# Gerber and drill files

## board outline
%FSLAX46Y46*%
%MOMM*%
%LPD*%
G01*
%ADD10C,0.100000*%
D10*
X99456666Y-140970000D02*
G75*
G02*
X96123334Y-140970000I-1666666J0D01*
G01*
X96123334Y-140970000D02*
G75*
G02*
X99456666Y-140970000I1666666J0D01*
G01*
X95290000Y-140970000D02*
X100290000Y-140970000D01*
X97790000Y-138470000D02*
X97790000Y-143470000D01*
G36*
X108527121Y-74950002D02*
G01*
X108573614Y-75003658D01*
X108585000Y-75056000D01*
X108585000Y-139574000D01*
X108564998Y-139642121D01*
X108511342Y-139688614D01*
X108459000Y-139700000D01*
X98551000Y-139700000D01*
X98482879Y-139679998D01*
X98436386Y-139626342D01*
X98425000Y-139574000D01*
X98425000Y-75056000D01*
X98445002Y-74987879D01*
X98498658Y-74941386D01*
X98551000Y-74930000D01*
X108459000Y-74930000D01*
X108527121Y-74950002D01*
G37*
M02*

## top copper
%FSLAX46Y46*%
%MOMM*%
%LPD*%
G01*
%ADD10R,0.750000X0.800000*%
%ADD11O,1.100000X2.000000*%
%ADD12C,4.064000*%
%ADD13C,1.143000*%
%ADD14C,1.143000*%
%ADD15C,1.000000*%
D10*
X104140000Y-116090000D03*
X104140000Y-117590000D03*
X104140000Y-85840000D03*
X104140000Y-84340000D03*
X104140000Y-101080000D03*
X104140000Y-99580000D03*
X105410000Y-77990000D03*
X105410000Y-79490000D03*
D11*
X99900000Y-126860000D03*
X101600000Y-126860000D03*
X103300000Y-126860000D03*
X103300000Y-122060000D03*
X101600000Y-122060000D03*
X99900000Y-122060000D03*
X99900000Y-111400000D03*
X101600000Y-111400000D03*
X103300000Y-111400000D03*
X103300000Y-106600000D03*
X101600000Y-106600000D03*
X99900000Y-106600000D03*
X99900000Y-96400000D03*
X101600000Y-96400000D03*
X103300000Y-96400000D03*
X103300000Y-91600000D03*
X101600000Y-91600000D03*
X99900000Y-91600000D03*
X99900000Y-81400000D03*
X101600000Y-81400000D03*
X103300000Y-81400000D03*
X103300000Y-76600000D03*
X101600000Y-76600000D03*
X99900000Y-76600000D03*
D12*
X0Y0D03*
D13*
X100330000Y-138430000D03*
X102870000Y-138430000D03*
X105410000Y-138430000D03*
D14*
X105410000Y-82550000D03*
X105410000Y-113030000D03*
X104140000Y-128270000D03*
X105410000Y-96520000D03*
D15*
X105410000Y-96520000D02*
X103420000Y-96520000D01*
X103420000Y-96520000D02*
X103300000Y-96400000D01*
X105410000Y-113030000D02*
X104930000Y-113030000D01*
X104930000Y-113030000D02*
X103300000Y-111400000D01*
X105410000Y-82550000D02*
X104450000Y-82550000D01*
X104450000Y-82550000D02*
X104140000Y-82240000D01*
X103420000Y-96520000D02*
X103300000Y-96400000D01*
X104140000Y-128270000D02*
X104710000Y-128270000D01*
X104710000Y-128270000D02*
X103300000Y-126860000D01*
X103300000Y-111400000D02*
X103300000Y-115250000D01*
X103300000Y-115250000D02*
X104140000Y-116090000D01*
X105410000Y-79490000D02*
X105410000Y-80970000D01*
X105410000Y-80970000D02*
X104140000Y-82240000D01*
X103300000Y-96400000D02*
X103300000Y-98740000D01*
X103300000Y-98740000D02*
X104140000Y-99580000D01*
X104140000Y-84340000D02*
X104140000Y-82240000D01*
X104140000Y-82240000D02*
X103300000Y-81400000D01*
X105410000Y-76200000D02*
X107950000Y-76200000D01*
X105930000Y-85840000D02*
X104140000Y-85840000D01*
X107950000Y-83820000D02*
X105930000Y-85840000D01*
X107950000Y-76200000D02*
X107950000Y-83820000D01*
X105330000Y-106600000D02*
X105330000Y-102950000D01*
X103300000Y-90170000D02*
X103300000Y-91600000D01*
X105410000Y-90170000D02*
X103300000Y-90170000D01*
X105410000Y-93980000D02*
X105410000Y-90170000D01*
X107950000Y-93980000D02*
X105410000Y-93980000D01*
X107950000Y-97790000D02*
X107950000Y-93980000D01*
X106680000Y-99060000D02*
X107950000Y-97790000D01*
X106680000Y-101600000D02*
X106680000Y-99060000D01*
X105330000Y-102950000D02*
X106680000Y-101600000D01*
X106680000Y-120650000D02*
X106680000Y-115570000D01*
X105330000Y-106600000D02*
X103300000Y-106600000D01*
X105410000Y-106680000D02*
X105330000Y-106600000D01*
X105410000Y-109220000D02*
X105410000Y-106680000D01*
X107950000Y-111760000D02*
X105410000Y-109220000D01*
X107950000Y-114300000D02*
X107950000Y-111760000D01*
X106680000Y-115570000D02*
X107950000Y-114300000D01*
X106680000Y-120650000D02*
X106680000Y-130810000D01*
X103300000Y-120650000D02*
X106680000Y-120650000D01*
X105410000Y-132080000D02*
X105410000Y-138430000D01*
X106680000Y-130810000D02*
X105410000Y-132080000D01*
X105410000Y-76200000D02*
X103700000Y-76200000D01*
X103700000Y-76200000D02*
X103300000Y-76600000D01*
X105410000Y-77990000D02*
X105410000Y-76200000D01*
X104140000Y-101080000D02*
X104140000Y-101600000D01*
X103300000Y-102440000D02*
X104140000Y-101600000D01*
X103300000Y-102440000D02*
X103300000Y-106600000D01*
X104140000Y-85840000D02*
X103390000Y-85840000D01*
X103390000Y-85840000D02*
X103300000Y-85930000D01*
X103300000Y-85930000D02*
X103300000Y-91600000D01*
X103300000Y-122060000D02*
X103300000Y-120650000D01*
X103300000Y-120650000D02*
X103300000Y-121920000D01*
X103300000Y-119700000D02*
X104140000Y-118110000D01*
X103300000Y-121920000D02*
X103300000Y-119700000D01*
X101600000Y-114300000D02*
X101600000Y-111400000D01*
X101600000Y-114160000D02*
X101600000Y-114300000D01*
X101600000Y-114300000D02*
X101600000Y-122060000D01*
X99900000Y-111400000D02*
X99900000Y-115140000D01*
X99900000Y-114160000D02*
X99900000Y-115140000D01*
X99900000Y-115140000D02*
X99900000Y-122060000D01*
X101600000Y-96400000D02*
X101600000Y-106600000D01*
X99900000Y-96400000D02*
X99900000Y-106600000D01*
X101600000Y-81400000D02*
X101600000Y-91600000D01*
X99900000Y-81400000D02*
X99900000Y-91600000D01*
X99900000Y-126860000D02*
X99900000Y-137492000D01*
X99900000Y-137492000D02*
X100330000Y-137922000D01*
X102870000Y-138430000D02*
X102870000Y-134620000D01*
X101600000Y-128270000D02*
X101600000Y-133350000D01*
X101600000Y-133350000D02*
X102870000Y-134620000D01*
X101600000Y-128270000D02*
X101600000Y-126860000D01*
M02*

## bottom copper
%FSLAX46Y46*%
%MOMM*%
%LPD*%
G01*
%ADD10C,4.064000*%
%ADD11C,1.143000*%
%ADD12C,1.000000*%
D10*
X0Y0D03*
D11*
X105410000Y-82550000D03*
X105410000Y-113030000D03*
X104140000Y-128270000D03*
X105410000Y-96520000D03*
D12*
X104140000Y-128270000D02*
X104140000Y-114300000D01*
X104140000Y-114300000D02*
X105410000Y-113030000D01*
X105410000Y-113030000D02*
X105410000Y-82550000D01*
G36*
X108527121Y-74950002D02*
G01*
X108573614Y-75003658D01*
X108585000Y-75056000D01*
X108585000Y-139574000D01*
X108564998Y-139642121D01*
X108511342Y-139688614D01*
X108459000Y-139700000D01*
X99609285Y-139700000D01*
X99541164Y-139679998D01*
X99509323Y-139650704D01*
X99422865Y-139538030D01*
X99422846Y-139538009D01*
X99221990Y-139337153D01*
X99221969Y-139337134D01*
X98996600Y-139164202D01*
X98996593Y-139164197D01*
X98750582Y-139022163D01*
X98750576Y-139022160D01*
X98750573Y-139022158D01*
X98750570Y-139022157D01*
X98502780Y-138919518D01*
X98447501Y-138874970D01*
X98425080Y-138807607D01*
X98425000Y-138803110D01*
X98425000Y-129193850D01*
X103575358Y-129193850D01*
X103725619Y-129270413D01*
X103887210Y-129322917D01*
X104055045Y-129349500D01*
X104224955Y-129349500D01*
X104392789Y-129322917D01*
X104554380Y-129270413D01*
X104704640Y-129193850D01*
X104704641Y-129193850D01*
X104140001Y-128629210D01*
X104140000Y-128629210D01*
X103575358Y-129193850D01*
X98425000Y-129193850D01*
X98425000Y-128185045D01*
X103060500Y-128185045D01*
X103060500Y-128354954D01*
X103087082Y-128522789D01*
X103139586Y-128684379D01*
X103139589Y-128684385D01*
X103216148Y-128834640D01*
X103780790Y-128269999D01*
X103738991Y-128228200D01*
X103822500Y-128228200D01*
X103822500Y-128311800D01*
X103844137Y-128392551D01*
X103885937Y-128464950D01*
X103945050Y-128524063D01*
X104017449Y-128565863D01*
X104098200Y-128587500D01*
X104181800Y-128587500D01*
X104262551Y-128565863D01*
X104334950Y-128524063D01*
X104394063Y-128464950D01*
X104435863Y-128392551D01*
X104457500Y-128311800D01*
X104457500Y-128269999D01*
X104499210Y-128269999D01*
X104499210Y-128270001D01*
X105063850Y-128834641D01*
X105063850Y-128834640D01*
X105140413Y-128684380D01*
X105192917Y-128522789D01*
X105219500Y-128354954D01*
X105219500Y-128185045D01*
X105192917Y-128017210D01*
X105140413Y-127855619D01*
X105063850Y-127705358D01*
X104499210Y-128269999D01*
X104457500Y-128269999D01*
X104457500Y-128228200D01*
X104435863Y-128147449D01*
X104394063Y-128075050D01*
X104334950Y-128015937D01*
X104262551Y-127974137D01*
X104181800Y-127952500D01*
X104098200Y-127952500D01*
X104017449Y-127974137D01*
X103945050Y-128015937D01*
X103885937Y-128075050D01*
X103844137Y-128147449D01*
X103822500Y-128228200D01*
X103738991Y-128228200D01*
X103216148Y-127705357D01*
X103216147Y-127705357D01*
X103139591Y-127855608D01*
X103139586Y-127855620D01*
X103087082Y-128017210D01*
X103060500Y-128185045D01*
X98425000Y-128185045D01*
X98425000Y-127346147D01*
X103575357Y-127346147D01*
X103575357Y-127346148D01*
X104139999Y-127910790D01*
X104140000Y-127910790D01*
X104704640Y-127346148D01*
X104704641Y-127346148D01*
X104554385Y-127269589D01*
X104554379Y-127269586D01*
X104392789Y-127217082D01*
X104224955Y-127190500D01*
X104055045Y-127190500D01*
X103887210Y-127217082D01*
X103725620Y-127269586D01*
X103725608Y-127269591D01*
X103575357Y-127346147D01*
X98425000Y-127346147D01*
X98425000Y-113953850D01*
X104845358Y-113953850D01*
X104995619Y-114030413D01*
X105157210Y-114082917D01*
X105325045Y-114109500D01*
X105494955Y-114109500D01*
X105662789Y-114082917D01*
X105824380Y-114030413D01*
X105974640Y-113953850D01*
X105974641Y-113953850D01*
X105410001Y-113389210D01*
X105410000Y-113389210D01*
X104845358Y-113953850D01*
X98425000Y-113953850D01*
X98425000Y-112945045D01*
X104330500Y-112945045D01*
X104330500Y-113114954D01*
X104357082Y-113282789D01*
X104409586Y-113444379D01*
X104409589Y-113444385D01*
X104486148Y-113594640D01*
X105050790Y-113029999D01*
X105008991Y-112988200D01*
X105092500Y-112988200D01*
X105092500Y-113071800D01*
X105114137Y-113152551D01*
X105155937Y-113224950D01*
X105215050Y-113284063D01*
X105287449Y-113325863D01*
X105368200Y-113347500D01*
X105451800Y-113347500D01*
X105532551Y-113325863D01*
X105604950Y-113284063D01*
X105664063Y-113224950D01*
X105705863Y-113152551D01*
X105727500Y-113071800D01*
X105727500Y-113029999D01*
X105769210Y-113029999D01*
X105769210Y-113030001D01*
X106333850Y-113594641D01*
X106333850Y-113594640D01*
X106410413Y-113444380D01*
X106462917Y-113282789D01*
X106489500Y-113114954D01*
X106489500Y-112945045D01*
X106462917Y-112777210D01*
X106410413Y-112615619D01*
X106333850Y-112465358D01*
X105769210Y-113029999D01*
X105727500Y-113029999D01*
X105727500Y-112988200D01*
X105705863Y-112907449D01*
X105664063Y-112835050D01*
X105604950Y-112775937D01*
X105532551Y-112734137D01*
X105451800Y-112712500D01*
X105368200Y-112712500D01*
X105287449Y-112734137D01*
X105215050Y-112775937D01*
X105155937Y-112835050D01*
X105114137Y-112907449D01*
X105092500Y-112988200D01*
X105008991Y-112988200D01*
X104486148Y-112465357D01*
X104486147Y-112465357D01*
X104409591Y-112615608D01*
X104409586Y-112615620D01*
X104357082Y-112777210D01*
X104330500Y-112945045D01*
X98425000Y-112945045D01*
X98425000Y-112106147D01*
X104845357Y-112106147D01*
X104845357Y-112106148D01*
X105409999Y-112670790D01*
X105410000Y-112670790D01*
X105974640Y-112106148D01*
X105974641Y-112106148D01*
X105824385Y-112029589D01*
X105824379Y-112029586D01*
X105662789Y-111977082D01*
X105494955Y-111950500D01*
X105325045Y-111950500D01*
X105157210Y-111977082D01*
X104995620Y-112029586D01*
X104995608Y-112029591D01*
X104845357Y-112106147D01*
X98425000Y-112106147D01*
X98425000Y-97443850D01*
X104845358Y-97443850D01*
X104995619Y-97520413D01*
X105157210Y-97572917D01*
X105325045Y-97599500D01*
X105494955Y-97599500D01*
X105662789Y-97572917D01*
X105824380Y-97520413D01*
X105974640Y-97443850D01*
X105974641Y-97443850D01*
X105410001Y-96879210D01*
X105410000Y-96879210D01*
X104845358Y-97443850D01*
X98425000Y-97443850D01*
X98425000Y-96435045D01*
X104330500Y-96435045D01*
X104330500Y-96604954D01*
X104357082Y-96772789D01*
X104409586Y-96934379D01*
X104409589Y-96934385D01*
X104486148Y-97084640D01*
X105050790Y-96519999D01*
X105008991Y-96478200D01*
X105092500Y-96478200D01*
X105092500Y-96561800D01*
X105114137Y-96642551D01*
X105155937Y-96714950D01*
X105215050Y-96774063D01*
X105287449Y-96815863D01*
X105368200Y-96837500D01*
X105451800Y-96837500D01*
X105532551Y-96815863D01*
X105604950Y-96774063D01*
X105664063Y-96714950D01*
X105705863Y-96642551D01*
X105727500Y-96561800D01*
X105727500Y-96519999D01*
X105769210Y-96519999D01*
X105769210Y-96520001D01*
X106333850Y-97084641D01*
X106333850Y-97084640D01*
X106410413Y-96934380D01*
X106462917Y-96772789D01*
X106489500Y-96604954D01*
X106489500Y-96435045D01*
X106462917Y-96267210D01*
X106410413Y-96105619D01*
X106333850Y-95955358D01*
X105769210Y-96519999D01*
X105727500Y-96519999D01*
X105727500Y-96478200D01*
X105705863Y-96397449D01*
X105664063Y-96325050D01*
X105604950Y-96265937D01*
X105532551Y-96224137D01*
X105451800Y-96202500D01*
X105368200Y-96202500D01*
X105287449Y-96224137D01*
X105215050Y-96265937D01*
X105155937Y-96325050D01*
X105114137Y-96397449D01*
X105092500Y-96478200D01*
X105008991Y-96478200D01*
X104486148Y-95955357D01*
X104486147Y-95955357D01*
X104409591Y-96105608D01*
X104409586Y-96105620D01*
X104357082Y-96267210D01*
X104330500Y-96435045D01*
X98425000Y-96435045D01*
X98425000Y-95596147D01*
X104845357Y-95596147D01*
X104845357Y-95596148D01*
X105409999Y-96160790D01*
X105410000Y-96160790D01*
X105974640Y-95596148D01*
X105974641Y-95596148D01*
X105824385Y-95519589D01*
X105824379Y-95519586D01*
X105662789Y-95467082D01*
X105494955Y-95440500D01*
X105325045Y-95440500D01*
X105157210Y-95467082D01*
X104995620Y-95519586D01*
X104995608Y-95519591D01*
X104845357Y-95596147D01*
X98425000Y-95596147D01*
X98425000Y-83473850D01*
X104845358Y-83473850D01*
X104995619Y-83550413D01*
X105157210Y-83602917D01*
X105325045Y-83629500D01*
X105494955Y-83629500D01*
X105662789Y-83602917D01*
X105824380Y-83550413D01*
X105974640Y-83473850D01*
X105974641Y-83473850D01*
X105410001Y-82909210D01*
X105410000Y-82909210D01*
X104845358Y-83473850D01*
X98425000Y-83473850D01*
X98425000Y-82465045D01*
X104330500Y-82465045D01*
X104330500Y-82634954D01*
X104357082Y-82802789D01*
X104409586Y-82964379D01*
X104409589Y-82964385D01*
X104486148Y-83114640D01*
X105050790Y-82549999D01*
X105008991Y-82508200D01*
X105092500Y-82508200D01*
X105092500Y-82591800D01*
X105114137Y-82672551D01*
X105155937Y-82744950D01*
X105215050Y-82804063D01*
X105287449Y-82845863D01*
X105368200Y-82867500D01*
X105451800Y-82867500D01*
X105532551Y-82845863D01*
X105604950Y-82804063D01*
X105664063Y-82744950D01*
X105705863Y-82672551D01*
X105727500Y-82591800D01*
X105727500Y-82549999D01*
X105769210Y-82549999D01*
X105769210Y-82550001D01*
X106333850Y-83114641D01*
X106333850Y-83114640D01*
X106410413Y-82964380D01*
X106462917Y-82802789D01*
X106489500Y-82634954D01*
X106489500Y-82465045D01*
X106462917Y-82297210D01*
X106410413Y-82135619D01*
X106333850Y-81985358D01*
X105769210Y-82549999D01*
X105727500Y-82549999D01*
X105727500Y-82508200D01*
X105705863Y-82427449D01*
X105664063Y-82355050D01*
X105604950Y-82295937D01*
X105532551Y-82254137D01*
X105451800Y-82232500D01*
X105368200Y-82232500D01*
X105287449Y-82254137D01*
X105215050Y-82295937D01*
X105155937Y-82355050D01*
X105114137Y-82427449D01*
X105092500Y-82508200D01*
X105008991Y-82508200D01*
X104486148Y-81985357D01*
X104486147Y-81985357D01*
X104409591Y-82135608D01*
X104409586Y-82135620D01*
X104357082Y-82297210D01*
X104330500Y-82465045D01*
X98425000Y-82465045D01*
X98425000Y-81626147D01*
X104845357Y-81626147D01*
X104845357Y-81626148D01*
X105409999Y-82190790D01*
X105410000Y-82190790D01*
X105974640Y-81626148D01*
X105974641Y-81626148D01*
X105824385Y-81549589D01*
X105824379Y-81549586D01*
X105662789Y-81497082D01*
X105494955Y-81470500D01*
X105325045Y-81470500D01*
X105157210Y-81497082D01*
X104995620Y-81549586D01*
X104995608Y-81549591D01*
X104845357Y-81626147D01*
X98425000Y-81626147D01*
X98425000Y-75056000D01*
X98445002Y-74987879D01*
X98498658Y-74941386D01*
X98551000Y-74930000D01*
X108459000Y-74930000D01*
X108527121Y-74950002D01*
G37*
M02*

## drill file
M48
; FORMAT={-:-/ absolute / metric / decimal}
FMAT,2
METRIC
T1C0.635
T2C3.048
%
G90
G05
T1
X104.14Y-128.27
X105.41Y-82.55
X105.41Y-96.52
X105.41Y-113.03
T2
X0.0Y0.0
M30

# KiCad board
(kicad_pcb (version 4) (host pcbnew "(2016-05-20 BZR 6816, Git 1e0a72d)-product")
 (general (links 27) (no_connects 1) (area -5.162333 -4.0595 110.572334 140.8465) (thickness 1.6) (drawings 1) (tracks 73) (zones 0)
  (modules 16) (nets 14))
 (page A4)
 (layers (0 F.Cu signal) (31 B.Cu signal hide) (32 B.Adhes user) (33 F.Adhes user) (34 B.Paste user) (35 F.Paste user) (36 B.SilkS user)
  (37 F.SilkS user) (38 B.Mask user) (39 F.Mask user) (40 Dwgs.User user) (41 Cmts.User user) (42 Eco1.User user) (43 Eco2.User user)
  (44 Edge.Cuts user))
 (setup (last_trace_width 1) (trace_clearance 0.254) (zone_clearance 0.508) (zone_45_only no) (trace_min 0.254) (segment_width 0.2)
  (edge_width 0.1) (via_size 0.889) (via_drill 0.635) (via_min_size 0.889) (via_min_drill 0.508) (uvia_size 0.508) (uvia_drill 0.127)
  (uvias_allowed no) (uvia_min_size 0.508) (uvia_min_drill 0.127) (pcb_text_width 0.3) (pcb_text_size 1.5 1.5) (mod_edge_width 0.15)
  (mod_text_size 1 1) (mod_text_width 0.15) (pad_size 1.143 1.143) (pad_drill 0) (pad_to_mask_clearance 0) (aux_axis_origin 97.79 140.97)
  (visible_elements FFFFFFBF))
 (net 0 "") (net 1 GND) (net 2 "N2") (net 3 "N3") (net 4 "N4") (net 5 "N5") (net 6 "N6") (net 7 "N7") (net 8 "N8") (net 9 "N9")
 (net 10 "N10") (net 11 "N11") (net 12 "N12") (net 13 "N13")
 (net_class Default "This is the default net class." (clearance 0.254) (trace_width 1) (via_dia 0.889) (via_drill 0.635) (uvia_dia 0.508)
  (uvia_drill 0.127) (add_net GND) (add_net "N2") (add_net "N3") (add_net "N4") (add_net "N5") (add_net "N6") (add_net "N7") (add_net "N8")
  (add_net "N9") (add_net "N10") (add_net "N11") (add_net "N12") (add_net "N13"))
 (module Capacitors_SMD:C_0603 (layer F.Cu) (at 104.14 116.84 270)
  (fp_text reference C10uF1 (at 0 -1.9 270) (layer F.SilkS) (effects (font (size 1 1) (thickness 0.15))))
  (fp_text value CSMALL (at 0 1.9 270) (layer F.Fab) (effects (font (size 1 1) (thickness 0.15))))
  (pad 1 smd rect (at -0.75 0 270) (size 0.8 0.75) (layers F.Cu F.Paste F.Mask) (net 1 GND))
  (pad 2 smd rect (at 0.75 0 270) (size 0.8 0.75) (layers F.Cu F.Paste F.Mask) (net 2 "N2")))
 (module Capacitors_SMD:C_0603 (layer F.Cu) (at 104.14 85.09 90)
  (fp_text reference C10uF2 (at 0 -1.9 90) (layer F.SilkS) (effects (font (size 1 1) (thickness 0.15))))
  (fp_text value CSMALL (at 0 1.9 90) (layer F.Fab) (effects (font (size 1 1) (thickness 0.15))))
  (pad 1 smd rect (at -0.75 0 90) (size 0.8 0.75) (layers F.Cu F.Paste F.Mask) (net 2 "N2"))
  (pad 2 smd rect (at 0.75 0 90) (size 0.8 0.75) (layers F.Cu F.Paste F.Mask) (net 1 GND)))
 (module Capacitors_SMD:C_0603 (layer F.Cu) (at 104.14 100.33 90)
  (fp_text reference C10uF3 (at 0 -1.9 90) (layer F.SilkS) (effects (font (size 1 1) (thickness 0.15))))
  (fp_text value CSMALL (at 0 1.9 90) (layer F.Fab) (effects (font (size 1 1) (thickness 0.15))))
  (pad 1 smd rect (at -0.75 0 90) (size 0.8 0.75) (layers F.Cu F.Paste F.Mask) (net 2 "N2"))
  (pad 2 smd rect (at 0.75 0 90) (size 0.8 0.75) (layers F.Cu F.Paste F.Mask) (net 1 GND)))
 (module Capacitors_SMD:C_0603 (layer F.Cu) (at 105.41 78.74 270)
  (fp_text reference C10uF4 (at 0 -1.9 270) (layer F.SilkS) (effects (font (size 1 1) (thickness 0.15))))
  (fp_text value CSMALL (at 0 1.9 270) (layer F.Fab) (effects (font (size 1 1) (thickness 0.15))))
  (pad 1 smd rect (at -0.75 0 270) (size 0.8 0.75) (layers F.Cu F.Paste F.Mask) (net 2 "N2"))
  (pad 2 smd rect (at 0.75 0 270) (size 0.8 0.75) (layers F.Cu F.Paste F.Mask) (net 1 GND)))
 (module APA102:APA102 (layer F.Cu) (at 101.6 124.46 270)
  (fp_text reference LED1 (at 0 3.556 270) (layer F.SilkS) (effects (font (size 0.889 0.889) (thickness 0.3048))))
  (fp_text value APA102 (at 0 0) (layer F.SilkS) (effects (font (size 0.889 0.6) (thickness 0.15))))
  (pad 1 smd oval (at 2.4 1.7 270) (size 2 1.1) (layers F.Cu F.Paste F.Mask) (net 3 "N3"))
  (pad 2 smd oval (at 2.4 0 270) (size 2 1.1) (layers F.Cu F.Paste F.Mask) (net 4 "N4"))
  (pad 3 smd oval (at 2.4 -1.7 270) (size 2 1.1) (layers F.Cu F.Paste F.Mask) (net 1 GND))
  (pad 4 smd oval (at -2.4 -1.7 90) (size 2 1.1) (layers F.Cu F.Paste F.Mask) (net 2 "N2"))
  (pad 5 smd oval (at -2.4 0 90) (size 2 1.1) (layers F.Cu F.Paste F.Mask) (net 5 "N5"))
  (pad 6 smd oval (at -2.4 1.7 90) (size 2 1.1) (layers F.Cu F.Paste F.Mask) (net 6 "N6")))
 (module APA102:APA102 (layer F.Cu) (at 101.6 109 270)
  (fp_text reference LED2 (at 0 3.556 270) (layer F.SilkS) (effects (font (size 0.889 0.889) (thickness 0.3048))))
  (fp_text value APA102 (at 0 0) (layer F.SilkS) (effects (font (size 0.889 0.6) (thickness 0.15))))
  (pad 1 smd oval (at 2.4 1.7 270) (size 2 1.1) (layers F.Cu F.Paste F.Mask) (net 6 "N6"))
  (pad 2 smd oval (at 2.4 0 270) (size 2 1.1) (layers F.Cu F.Paste F.Mask) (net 5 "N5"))
  (pad 3 smd oval (at 2.4 -1.7 270) (size 2 1.1) (layers F.Cu F.Paste F.Mask) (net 1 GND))
  (pad 4 smd oval (at -2.4 -1.7 90) (size 2 1.1) (layers F.Cu F.Paste F.Mask) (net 2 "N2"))
  (pad 5 smd oval (at -2.4 0 90) (size 2 1.1) (layers F.Cu F.Paste F.Mask) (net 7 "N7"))
  (pad 6 smd oval (at -2.4 1.7 90) (size 2 1.1) (layers F.Cu F.Paste F.Mask) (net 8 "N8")))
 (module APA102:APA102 (layer F.Cu) (at 101.6 94 270)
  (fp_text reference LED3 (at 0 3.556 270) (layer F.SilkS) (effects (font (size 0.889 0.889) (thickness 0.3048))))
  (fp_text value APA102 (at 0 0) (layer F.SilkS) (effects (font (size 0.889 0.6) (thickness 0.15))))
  (pad 1 smd oval (at 2.4 1.7 270) (size 2 1.1) (layers F.Cu F.Paste F.Mask) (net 8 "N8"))
  (pad 2 smd oval (at 2.4 0 270) (size 2 1.1) (layers F.Cu F.Paste F.Mask) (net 7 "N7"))
  (pad 3 smd oval (at 2.4 -1.7 270) (size 2 1.1) (layers F.Cu F.Paste F.Mask) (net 1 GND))
  (pad 4 smd oval (at -2.4 -1.7 90) (size 2 1.1) (layers F.Cu F.Paste F.Mask) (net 2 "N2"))
  (pad 5 smd oval (at -2.4 0 90) (size 2 1.1) (layers F.Cu F.Paste F.Mask) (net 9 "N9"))
  (pad 6 smd oval (at -2.4 1.7 90) (size 2 1.1) (layers F.Cu F.Paste F.Mask) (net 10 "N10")))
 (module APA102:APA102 (layer F.Cu) (at 101.6 79 270)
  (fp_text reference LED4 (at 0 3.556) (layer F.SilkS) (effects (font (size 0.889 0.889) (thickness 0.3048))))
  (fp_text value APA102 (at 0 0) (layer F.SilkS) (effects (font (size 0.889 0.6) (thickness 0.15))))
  (pad 1 smd oval (at 2.4 1.7 270) (size 2 1.1) (layers F.Cu F.Paste F.Mask) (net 10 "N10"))
  (pad 2 smd oval (at 2.4 0 270) (size 2 1.1) (layers F.Cu F.Paste F.Mask) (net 9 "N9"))
  (pad 3 smd oval (at 2.4 -1.7 270) (size 2 1.1) (layers F.Cu F.Paste F.Mask) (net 1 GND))
  (pad 4 smd oval (at -2.4 -1.7 90) (size 2 1.1) (layers F.Cu F.Paste F.Mask) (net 2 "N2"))
  (pad 5 smd oval (at -2.4 0 90) (size 2 1.1) (layers F.Cu F.Paste F.Mask) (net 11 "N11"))
  (pad 6 smd oval (at -2.4 1.7 90) (size 2 1.1) (layers F.Cu F.Paste F.Mask) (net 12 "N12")))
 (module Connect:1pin (layer F.Cu) (at 0 0)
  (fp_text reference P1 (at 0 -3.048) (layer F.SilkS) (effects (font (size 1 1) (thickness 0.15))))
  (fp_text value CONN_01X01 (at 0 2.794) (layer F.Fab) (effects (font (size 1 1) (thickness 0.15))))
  (pad 1 thru_hole circle (at 0 0) (size 4.064 4.064) (drill 3.048) (layers *.Cu *.Mask F.SilkS) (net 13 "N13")))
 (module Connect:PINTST (layer F.Cu) (at 100.33 138.43)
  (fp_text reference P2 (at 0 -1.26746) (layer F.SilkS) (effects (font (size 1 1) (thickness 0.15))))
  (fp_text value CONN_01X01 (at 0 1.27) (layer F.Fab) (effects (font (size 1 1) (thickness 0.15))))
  (pad 1 smd circle (at 0 0) (size 1.143 1.143) (layers F.Cu F.Paste F.Mask) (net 3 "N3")))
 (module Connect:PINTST (layer F.Cu) (at 102.87 138.43)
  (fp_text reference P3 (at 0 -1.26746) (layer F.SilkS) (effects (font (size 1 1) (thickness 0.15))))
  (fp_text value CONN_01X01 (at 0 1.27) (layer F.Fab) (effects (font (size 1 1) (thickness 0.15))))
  (pad 1 smd circle (at 0 0) (size 1.143 1.143) (layers F.Cu F.Paste F.Mask) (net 4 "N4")))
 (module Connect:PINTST (layer F.Cu) (at 105.41 138.43)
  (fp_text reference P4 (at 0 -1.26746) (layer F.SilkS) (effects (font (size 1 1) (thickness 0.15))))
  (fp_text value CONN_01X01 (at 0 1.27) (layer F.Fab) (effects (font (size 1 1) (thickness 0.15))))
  (pad 1 smd circle (at 0 0) (size 1.143 1.143) (layers F.Cu F.Paste F.Mask) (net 2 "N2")))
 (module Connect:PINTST (layer F.Cu) (at 105.41 82.55)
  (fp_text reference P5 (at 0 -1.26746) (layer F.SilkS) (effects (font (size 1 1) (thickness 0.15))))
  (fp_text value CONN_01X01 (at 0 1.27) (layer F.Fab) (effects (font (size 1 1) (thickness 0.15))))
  (pad 1 thru_hole circle (at 0 0) (size 1.143 1.143) (drill 0.635) (layers *.Cu *.Mask F.SilkS) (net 1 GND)))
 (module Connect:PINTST (layer F.Cu) (at 105.41 113.03)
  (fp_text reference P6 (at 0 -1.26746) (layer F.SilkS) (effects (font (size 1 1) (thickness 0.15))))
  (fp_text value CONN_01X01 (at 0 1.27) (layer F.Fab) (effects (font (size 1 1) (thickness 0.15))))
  (pad 1 thru_hole circle (at 0 0) (size 1.143 1.143) (drill 0.635) (layers *.Cu *.Mask F.SilkS) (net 1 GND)))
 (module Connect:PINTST (layer F.Cu) (at 104.14 128.27)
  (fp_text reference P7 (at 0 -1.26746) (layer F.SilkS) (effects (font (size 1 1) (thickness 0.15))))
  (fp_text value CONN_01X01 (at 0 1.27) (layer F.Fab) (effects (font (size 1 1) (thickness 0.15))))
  (pad 1 thru_hole circle (at 0 0) (size 1.143 1.143) (drill 0.635) (layers *.Cu *.Mask F.SilkS) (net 1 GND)))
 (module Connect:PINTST (layer F.Cu) (at 105.41 96.52)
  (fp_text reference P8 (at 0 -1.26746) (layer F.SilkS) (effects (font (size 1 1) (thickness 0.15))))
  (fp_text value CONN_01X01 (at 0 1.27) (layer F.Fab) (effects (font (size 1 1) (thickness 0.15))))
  (pad 1 thru_hole circle (at 0 0) (size 1.143 1.143) (drill 0.635) (layers *.Cu *.Mask F.SilkS) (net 1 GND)))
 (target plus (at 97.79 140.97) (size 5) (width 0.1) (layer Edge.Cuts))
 (segment (start 104.14 128.27) (end 104.14 114.3) (width 1) (layer B.Cu) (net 1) (status 400000))
 (segment (start 104.14 114.3) (end 105.41 113.03) (width 1) (layer B.Cu) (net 1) (status 800000))
 (segment (start 105.41 113.03) (end 105.41 82.55) (width 1) (layer B.Cu) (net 1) (status C00000))
 (segment (start 105.41 96.52) (end 103.42 96.52) (width 1) (layer F.Cu) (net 1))
 (segment (start 103.42 96.52) (end 103.3 96.4) (width 1) (layer F.Cu) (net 1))
 (segment (start 105.41 113.03) (end 104.93 113.03) (width 1) (layer F.Cu) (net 1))
 (segment (start 104.93 113.03) (end 103.3 111.4) (width 1) (layer F.Cu) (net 1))
 (segment (start 105.41 82.55) (end 104.45 82.55) (width 1) (layer F.Cu) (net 1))
 (segment (start 104.45 82.55) (end 104.14 82.24) (width 1) (layer F.Cu) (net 1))
 (segment (start 103.42 96.52) (end 103.3 96.4) (width 1) (layer F.Cu) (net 1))
 (segment (start 104.14 128.27) (end 104.71 128.27) (width 1) (layer F.Cu) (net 1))
 (segment (start 104.71 128.27) (end 103.3 126.86) (width 1) (layer F.Cu) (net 1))
 (segment (start 103.3 111.4) (end 103.3 115.25) (width 1) (layer F.Cu) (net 1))
 (segment (start 103.3 115.25) (end 104.14 116.09) (width 1) (layer F.Cu) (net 1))
 (segment (start 105.41 79.49) (end 105.41 80.97) (width 1) (layer F.Cu) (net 1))
 (segment (start 105.41 80.97) (end 104.14 82.24) (width 1) (layer F.Cu) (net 1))
 (segment (start 103.3 96.4) (end 103.3 98.74) (width 1) (layer F.Cu) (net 1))
 (segment (start 103.3 98.74) (end 104.14 99.58) (width 1) (layer F.Cu) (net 1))
 (segment (start 104.14 84.34) (end 104.14 82.24) (width 1) (layer F.Cu) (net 1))
 (segment (start 104.14 82.24) (end 103.3 81.4) (width 1) (layer F.Cu) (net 1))
 (segment (start 105.41 76.2) (end 107.95 76.2) (width 1) (layer F.Cu) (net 2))
 (segment (start 105.93 85.84) (end 104.14 85.84) (width 1) (layer F.Cu) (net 2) (status 800000))
 (segment (start 107.95 83.82) (end 105.93 85.84) (width 1) (layer F.Cu) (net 2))
 (segment (start 107.95 76.2) (end 107.95 83.82) (width 1) (layer F.Cu) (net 2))
 (segment (start 105.33 106.6) (end 105.33 102.95) (width 1) (layer F.Cu) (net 2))
 (segment (start 103.3 90.17) (end 103.3 91.6) (width 1) (layer F.Cu) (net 2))
 (segment (start 105.41 90.17) (end 103.3 90.17) (width 1) (layer F.Cu) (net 2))
 (segment (start 105.41 93.98) (end 105.41 90.17) (width 1) (layer F.Cu) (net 2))
 (segment (start 107.95 93.98) (end 105.41 93.98) (width 1) (layer F.Cu) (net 2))
 (segment (start 107.95 97.79) (end 107.95 93.98) (width 1) (layer F.Cu) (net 2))
 (segment (start 106.68 99.06) (end 107.95 97.79) (width 1) (layer F.Cu) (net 2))
 (segment (start 106.68 101.6) (end 106.68 99.06) (width 1) (layer F.Cu) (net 2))
 (segment (start 105.33 102.95) (end 106.68 101.6) (width 1) (layer F.Cu) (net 2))
 (segment (start 106.68 120.65) (end 106.68 115.57) (width 1) (layer F.Cu) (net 2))
 (segment (start 105.33 106.6) (end 103.3 106.6) (width 1) (layer F.Cu) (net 2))
 (segment (start 105.41 106.68) (end 105.33 106.6) (width 1) (layer F.Cu) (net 2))
 (segment (start 105.41 109.22) (end 105.41 106.68) (width 1) (layer F.Cu) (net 2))
 (segment (start 107.95 111.76) (end 105.41 109.22) (width 1) (layer F.Cu) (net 2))
 (segment (start 107.95 114.3) (end 107.95 111.76) (width 1) (layer F.Cu) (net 2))
 (segment (start 106.68 115.57) (end 107.95 114.3) (width 1) (layer F.Cu) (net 2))
 (segment (start 106.68 120.65) (end 106.68 130.81) (width 1) (layer F.Cu) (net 2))
 (segment (start 103.3 120.65) (end 106.68 120.65) (width 1) (layer F.Cu) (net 2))
 (segment (start 105.41 132.08) (end 105.41 138.43) (width 1) (layer F.Cu) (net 2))
 (segment (start 106.68 130.81) (end 105.41 132.08) (width 1) (layer F.Cu) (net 2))
 (segment (start 105.41 76.2) (end 103.7 76.2) (width 1) (layer F.Cu) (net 2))
 (segment (start 103.7 76.2) (end 103.3 76.6) (width 1) (layer F.Cu) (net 2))
 (segment (start 105.41 77.99) (end 105.41 76.2) (width 1) (layer F.Cu) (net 2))
 (segment (start 104.14 101.08) (end 104.14 101.6) (width 1) (layer F.Cu) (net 2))
 (segment (start 103.3 102.44) (end 104.14 101.6) (width 1) (layer F.Cu) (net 2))
 (segment (start 103.3 102.44) (end 103.3 106.6) (width 1) (layer F.Cu) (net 2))
 (segment (start 104.14 85.84) (end 103.39 85.84) (width 1) (layer F.Cu) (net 2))
 (segment (start 103.39 85.84) (end 103.3 85.93) (width 1) (layer F.Cu) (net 2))
 (segment (start 103.3 85.93) (end 103.3 91.6) (width 1) (layer F.Cu) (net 2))
 (segment (start 103.3 122.06) (end 103.3 120.65) (width 1) (layer F.Cu) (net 2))
 (segment (start 103.3 120.65) (end 103.3 121.92) (width 1) (layer F.Cu) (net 2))
 (segment (start 103.3 119.7) (end 104.14 118.11) (width 1) (layer F.Cu) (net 2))
 (segment (start 103.3 121.92) (end 103.3 119.7) (width 1) (layer F.Cu) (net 2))
 (segment (start 101.6 114.3) (end 101.6 111.4) (width 1) (layer F.Cu) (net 5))
 (segment (start 101.6 114.16) (end 101.6 114.3) (width 1) (layer F.Cu) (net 5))
 (segment (start 101.6 114.3) (end 101.6 122.06) (width 1) (layer F.Cu) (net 5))
 (segment (start 99.9 111.4) (end 99.9 115.14) (width 1) (layer F.Cu) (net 6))
 (segment (start 99.9 114.16) (end 99.9 115.14) (width 1) (layer F.Cu) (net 6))
 (segment (start 99.9 115.14) (end 99.9 122.06) (width 1) (layer F.Cu) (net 6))
 (segment (start 101.6 96.4) (end 101.6 106.6) (width 1) (layer F.Cu) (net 7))
 (segment (start 99.9 96.4) (end 99.9 106.6) (width 1) (layer F.Cu) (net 8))
 (segment (start 101.6 81.4) (end 101.6 91.6) (width 1) (layer F.Cu) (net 9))
 (segment (start 99.9 81.4) (end 99.9 91.6) (width 1) (layer F.Cu) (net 10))
 (segment (start 99.9 126.86) (end 99.9 137.492) (width 1) (layer F.Cu) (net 3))
 (segment (start 99.9 137.492) (end 100.33 137.922) (width 1) (layer F.Cu) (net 3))
 (segment (start 102.87 138.43) (end 102.87 134.62) (width 1) (layer F.Cu) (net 4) (status 400000))
 (segment (start 101.6 128.27) (end 101.6 133.35) (width 1) (layer F.Cu) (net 4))
 (segment (start 101.6 133.35) (end 102.87 134.62) (width 1) (layer F.Cu) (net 4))
 (segment (start 101.6 128.27) (end 101.6 126.86) (width 1) (layer F.Cu) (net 4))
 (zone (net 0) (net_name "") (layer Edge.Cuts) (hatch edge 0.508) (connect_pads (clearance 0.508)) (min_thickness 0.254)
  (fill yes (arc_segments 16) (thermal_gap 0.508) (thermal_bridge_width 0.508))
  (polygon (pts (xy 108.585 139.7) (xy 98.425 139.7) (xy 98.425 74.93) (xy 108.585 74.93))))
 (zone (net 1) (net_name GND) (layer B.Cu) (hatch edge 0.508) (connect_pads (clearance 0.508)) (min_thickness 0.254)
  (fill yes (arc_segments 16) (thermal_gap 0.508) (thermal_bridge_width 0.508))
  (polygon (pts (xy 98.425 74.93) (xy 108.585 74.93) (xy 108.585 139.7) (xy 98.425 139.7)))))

